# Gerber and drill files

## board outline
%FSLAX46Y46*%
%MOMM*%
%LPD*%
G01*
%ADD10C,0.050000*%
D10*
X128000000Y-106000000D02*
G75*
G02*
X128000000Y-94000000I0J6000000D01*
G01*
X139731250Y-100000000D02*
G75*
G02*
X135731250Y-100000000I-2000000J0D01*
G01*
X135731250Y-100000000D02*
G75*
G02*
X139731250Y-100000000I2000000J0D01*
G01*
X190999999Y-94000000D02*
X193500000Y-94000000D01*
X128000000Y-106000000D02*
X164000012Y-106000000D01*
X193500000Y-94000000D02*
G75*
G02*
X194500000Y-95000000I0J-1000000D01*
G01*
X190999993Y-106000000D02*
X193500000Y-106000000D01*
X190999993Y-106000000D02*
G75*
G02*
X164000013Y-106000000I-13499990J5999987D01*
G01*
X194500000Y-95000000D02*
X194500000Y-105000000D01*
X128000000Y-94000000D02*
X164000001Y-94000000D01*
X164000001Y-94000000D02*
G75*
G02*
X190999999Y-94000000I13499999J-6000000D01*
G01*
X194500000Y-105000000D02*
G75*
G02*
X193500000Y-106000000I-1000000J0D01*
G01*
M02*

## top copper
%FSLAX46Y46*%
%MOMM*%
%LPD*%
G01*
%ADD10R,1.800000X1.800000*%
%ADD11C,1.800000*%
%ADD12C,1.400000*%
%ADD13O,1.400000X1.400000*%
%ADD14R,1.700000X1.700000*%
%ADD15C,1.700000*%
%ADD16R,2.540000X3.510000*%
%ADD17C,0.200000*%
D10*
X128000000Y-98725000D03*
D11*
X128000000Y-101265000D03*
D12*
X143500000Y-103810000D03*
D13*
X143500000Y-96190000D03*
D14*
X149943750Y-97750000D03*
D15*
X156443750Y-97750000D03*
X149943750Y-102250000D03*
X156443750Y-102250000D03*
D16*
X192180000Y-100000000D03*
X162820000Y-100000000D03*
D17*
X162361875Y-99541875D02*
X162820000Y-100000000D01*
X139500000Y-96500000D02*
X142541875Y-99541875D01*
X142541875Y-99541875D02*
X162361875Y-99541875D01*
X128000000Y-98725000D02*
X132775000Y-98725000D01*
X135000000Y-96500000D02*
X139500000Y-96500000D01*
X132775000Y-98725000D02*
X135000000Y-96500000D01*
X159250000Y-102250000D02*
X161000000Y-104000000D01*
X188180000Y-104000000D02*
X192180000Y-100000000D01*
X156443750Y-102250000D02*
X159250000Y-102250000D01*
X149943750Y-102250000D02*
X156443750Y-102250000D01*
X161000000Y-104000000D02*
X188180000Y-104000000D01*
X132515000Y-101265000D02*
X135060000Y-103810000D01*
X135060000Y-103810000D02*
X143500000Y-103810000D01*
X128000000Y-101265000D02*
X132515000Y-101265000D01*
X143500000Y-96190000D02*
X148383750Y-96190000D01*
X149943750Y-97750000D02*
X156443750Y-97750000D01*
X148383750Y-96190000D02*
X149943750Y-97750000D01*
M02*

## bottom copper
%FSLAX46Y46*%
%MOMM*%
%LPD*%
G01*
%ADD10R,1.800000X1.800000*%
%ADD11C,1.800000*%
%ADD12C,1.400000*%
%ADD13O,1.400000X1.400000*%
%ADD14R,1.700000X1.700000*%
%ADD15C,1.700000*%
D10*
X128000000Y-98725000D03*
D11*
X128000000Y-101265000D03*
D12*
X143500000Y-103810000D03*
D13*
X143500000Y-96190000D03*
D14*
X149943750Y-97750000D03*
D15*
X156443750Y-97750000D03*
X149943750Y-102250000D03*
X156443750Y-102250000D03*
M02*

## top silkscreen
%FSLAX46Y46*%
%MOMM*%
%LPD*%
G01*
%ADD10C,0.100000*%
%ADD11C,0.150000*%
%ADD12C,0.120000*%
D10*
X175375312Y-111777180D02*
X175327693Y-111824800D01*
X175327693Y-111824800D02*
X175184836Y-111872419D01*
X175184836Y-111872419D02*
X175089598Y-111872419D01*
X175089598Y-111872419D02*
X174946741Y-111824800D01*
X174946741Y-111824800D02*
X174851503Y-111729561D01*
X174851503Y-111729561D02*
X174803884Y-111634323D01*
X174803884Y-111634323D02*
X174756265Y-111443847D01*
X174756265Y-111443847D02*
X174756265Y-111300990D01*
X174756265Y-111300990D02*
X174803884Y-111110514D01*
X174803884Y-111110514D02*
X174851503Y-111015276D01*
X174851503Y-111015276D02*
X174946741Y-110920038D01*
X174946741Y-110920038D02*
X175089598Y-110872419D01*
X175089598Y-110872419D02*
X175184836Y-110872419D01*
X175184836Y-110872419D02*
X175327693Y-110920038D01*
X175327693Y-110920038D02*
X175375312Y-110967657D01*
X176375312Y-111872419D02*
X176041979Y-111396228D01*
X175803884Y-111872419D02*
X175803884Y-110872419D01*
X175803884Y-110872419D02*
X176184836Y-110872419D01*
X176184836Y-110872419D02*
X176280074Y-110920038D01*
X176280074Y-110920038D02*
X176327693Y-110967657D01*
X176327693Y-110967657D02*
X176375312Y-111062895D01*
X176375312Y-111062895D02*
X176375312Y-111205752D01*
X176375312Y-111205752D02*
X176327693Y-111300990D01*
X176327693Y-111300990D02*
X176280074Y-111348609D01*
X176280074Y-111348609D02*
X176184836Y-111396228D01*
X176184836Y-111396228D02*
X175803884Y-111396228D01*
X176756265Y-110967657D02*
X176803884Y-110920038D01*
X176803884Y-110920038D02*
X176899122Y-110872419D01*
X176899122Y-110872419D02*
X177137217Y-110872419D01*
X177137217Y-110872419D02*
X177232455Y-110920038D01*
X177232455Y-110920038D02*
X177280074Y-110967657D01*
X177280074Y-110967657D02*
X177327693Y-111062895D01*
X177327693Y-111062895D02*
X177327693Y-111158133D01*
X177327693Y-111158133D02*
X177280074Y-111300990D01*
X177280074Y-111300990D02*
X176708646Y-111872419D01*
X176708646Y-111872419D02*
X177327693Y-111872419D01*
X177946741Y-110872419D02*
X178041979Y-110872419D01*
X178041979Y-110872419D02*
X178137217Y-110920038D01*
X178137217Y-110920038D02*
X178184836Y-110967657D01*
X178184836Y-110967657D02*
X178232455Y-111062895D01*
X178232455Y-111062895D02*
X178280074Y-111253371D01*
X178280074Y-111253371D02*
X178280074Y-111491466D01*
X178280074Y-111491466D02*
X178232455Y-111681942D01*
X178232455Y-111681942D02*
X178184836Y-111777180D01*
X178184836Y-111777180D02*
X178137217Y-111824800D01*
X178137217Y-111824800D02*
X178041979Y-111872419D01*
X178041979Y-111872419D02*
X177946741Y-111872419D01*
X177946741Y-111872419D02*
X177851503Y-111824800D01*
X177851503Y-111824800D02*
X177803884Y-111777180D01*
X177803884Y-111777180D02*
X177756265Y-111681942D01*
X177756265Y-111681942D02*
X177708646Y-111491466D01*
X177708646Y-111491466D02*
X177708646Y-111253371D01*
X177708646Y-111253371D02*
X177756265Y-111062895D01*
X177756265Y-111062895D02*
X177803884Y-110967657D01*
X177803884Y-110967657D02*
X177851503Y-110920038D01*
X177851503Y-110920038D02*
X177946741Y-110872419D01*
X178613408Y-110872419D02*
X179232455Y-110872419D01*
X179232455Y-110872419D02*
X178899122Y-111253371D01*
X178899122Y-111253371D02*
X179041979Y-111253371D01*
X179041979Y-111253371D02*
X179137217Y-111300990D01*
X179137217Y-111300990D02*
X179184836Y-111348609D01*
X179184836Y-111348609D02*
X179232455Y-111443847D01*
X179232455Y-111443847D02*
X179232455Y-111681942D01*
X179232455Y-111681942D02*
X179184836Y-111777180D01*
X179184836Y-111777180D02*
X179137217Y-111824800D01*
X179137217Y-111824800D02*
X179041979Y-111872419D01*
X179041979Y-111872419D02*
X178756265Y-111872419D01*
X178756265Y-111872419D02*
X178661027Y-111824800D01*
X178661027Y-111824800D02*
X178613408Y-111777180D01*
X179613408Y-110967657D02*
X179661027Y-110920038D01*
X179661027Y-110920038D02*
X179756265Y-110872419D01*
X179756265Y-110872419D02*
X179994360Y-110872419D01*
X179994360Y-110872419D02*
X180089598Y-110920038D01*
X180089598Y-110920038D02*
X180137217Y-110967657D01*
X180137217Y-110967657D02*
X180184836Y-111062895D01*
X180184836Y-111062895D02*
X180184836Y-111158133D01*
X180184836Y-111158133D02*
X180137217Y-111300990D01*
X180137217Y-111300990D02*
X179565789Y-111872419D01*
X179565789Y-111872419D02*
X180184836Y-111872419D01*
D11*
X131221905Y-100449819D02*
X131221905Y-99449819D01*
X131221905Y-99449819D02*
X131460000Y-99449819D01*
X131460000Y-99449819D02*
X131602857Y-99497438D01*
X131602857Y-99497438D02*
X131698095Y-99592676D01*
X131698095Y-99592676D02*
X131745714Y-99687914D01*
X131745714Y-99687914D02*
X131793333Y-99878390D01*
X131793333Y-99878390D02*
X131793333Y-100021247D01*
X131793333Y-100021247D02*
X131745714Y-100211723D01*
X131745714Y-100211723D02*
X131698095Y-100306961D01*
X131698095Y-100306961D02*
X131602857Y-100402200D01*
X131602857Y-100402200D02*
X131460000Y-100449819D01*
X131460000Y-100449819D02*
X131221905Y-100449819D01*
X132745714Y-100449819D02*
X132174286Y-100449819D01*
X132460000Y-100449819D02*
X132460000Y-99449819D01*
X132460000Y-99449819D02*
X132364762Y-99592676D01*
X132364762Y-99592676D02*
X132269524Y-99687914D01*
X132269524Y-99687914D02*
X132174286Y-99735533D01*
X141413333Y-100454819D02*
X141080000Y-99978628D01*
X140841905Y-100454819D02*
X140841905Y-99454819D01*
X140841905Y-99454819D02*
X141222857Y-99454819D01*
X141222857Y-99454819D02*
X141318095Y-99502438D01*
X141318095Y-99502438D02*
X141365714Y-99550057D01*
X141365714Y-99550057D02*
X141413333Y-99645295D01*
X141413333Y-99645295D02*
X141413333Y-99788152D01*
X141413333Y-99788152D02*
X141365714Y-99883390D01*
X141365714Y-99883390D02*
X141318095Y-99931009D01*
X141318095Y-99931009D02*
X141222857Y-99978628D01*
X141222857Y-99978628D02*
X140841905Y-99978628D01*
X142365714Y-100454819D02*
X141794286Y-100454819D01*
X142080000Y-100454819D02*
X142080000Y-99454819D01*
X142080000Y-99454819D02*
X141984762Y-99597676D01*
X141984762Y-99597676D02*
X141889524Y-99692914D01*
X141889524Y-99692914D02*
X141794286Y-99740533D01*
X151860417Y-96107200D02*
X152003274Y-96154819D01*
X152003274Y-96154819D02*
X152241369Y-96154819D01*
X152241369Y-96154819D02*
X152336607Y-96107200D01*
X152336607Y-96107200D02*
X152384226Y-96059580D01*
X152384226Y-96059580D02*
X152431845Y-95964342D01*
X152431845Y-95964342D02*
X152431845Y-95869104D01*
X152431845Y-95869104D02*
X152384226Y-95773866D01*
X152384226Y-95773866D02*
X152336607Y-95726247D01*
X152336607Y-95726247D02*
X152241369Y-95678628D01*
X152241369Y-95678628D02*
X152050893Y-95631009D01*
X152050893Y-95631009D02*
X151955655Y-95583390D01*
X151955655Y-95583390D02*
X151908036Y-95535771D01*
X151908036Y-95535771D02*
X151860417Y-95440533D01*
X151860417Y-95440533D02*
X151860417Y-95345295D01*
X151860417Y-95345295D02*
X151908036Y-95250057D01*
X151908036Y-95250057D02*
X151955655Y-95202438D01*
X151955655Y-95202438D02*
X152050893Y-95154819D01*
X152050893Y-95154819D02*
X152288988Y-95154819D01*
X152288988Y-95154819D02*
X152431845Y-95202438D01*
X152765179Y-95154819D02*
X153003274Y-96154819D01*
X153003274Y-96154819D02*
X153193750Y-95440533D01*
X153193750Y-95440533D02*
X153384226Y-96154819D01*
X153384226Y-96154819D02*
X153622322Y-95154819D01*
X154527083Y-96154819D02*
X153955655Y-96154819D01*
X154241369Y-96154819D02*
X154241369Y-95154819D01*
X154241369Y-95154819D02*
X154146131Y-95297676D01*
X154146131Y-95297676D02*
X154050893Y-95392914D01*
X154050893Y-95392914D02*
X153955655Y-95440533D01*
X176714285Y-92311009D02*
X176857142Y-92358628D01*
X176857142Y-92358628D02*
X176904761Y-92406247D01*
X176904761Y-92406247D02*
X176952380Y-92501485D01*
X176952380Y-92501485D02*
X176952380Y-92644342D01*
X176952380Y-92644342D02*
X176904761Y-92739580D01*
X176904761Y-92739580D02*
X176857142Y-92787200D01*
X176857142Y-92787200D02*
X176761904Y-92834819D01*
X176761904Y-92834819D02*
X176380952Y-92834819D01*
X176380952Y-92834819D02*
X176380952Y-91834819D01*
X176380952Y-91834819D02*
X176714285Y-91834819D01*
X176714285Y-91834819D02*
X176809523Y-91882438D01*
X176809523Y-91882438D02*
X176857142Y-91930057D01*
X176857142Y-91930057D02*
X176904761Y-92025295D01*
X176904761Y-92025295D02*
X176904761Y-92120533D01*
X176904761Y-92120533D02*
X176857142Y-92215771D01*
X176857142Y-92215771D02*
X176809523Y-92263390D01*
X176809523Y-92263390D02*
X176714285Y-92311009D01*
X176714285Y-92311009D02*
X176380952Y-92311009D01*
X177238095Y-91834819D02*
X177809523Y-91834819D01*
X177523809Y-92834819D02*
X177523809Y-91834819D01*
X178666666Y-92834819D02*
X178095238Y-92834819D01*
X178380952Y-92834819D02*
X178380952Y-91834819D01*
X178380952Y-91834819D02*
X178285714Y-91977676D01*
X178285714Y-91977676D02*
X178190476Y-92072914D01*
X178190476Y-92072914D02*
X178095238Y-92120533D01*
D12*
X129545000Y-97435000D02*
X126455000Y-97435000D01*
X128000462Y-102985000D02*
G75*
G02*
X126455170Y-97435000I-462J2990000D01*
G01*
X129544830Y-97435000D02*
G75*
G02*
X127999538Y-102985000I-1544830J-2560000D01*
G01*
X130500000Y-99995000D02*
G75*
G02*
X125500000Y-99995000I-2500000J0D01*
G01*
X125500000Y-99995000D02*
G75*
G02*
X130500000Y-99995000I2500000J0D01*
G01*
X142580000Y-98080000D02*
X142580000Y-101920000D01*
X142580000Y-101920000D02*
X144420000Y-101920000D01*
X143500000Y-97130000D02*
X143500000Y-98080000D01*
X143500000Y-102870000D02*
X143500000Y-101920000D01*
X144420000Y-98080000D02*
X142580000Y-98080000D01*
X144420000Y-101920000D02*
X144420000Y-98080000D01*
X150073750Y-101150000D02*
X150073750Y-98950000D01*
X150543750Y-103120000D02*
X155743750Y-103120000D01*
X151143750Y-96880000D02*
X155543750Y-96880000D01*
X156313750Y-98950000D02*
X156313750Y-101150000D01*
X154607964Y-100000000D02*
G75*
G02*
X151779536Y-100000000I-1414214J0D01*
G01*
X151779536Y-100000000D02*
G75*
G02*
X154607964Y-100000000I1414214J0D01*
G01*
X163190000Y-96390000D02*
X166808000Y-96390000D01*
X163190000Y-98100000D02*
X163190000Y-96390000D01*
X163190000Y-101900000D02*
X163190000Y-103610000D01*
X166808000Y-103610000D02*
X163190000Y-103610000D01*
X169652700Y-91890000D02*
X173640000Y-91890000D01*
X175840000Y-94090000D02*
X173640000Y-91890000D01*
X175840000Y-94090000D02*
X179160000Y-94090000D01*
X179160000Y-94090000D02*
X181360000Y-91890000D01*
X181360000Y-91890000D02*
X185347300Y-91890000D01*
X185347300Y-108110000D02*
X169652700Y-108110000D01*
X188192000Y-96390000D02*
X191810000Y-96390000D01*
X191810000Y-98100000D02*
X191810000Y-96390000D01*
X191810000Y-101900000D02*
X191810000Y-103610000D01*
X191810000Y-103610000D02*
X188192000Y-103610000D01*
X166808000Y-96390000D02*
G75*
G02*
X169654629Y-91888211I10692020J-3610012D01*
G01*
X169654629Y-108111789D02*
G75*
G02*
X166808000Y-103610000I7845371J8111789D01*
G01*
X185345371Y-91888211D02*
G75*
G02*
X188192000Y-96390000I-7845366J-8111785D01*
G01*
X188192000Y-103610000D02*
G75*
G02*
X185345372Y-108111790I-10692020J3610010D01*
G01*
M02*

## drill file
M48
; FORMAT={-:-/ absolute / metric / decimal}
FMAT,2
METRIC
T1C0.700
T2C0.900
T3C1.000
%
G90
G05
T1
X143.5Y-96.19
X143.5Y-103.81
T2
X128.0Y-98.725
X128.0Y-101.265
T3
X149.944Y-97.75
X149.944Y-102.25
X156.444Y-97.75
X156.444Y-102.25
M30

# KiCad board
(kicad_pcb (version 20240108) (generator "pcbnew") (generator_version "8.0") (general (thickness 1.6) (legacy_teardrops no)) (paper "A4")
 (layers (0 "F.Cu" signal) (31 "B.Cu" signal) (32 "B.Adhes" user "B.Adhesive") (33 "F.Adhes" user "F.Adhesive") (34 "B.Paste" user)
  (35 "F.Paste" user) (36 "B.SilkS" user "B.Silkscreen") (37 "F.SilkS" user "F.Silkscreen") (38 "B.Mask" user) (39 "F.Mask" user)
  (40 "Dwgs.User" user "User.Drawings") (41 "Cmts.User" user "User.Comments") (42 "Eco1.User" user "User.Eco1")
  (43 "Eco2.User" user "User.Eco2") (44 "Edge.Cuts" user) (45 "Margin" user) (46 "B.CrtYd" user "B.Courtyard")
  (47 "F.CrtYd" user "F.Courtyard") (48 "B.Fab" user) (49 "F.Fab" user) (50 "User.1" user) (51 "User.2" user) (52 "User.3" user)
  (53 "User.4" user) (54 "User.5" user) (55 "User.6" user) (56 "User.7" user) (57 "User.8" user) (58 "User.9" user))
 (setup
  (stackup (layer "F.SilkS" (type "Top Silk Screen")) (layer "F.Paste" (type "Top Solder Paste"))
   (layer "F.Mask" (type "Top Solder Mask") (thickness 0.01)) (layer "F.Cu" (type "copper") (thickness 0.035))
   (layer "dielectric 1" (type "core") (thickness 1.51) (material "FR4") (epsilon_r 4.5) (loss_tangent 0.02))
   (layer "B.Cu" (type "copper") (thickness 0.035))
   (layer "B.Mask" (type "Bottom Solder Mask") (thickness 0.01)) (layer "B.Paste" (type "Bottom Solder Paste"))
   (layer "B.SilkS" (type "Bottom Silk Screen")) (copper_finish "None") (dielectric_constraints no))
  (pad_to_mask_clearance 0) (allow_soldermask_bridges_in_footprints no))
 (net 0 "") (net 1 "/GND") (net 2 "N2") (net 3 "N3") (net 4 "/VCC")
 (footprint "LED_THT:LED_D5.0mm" (layer "F.Cu") (at 128 98.725 -90)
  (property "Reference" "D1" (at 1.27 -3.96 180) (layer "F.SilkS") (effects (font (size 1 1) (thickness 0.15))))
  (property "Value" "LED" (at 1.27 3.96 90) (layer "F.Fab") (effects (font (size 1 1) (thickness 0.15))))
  (fp_line (start -1.29 -1.545) (end -1.29 1.545) (stroke (width 0.12) (type solid)) (layer "F.SilkS"))
  (fp_arc (start 4.26 -0.000462) (mid 2.072002 2.880433) (end -1.29 1.54483) (stroke (width 0.12) (type solid)) (layer "F.SilkS"))
  (fp_arc (start -1.29 -1.54483) (mid 2.072002 -2.880433) (end 4.26 0.000462) (stroke (width 0.12) (type solid)) (layer "F.SilkS"))
  (fp_circle (center 1.27 0) (end 3.77 0) (stroke (width 0.12) (type solid)) (fill none) (layer "F.SilkS"))
  (pad "1" thru_hole rect (at 0 0 270) (size 1.8 1.8) (drill 0.9) (layers "*.Cu" "*.Mask") (remove_unused_layers no) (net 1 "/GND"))
  (pad "2" thru_hole circle (at 2.54 0 270) (size 1.8 1.8) (drill 0.9) (layers "*.Cu" "*.Mask") (remove_unused_layers no) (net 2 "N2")))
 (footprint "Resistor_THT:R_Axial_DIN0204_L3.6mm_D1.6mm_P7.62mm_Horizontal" (layer "F.Cu") (at 143.5 103.81 90)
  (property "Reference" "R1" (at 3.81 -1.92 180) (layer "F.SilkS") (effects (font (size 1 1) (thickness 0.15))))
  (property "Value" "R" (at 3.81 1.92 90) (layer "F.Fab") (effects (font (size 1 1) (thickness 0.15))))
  (fp_line (start 5.73 -0.92) (end 1.89 -0.92) (stroke (width 0.12) (type solid)) (layer "F.SilkS"))
  (fp_line (start 1.89 -0.92) (end 1.89 0.92) (stroke (width 0.12) (type solid)) (layer "F.SilkS"))
  (fp_line (start 6.68 0) (end 5.73 0) (stroke (width 0.12) (type solid)) (layer "F.SilkS"))
  (fp_line (start 0.94 0) (end 1.89 0) (stroke (width 0.12) (type solid)) (layer "F.SilkS"))
  (fp_line (start 5.73 0.92) (end 5.73 -0.92) (stroke (width 0.12) (type solid)) (layer "F.SilkS"))
  (fp_line (start 1.89 0.92) (end 5.73 0.92) (stroke (width 0.12) (type solid)) (layer "F.SilkS"))
  (pad "1" thru_hole circle (at 0 0 90) (size 1.4 1.4) (drill 0.7) (layers "*.Cu" "*.Mask") (remove_unused_layers no) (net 2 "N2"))
  (pad "2" thru_hole oval (at 7.62 0 90) (size 1.4 1.4) (drill 0.7) (layers "*.Cu" "*.Mask") (remove_unused_layers no) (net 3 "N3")))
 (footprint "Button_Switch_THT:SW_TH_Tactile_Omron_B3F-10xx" (layer "F.Cu") (at 149.94375 97.75)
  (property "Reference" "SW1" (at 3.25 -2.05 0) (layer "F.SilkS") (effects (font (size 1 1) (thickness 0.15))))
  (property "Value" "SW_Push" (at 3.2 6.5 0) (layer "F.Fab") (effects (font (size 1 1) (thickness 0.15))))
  (fp_line (start 0.13 3.4) (end 0.13 1.2) (stroke (width 0.12) (type solid)) (layer "F.SilkS"))
  (fp_line (start 0.6 5.37) (end 5.8 5.37) (stroke (width 0.12) (type solid)) (layer "F.SilkS"))
  (fp_line (start 1.2 -0.87) (end 5.6 -0.87) (stroke (width 0.12) (type solid)) (layer "F.SilkS"))
  (fp_line (start 6.37 1.2) (end 6.37 3.4) (stroke (width 0.12) (type solid)) (layer "F.SilkS"))
  (fp_circle (center 3.25 2.25) (end 4.25 3.25) (stroke (width 0.12) (type solid)) (fill none) (layer "F.SilkS"))
  (pad "1" thru_hole rect (at 0 0) (size 1.7 1.7) (drill 1) (layers "*.Cu" "*.Mask") (remove_unused_layers no) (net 3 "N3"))
  (pad "1" thru_hole circle (at 6.5 0) (size 1.7 1.7) (drill 1) (layers "*.Cu" "*.Mask") (remove_unused_layers no) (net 3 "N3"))
  (pad "2" thru_hole circle (at 0 4.5) (size 1.7 1.7) (drill 1) (layers "*.Cu" "*.Mask") (remove_unused_layers no) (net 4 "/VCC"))
  (pad "2" thru_hole circle (at 6.5 4.5) (size 1.7 1.7) (drill 1) (layers "*.Cu" "*.Mask") (remove_unused_layers no) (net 4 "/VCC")))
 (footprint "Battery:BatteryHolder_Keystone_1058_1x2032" (layer "F.Cu") (at 177.5 100 180)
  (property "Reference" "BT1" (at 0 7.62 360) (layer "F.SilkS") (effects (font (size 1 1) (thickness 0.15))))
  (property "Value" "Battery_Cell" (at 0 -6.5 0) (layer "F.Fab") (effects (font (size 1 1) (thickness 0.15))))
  (fp_line (start 14.31 3.61) (end 10.692 3.61) (stroke (width 0.12) (type solid)) (layer "F.SilkS"))
  (fp_line (start 14.31 1.9) (end 14.31 3.61) (stroke (width 0.12) (type solid)) (layer "F.SilkS"))
  (fp_line (start 14.31 -1.9) (end 14.31 -3.61) (stroke (width 0.12) (type solid)) (layer "F.SilkS"))
  (fp_line (start 10.692 -3.61) (end 14.31 -3.61) (stroke (width 0.12) (type solid)) (layer "F.SilkS"))
  (fp_line (start 7.8473 8.11) (end 3.86 8.11) (stroke (width 0.12) (type solid)) (layer "F.SilkS"))
  (fp_line (start 1.66 5.91) (end 3.86 8.11) (stroke (width 0.12) (type solid)) (layer "F.SilkS"))
  (fp_line (start 1.66 5.91) (end -1.66 5.91) (stroke (width 0.12) (type solid)) (layer "F.SilkS"))
  (fp_line (start -1.66 5.91) (end -3.86 8.11) (stroke (width 0.12) (type solid)) (layer "F.SilkS"))
  (fp_line (start -3.86 8.11) (end -7.8473 8.11) (stroke (width 0.12) (type solid)) (layer "F.SilkS"))
  (fp_line (start -7.8473 -8.11) (end 7.8473 -8.11) (stroke (width 0.12) (type solid)) (layer "F.SilkS"))
  (fp_line (start -10.692 3.61) (end -14.31 3.61) (stroke (width 0.12) (type solid)) (layer "F.SilkS"))
  (fp_line (start -14.31 1.9) (end -14.31 3.61) (stroke (width 0.12) (type solid)) (layer "F.SilkS"))
  (fp_line (start -14.31 -1.9) (end -14.31 -3.61) (stroke (width 0.12) (type solid)) (layer "F.SilkS"))
  (fp_line (start -14.31 -3.61) (end -10.692 -3.61) (stroke (width 0.12) (type solid)) (layer "F.SilkS"))
  (fp_arc (start 10.692 3.61) (mid 9.538084 6.031244) (end 7.845371 8.111789) (stroke (width 0.12) (type solid)) (layer "F.SilkS"))
  (fp_arc (start 7.845371 -8.111789) (mid 9.538085 -6.031244) (end 10.692 -3.61) (stroke (width 0.12) (type solid)) (layer "F.SilkS"))
  (fp_arc (start -7.845371 8.111789) (mid -9.538085 6.031244) (end -10.692 3.61) (stroke (width 0.12) (type solid)) (layer "F.SilkS"))
  (fp_arc (start -10.692 -3.61) (mid -9.538084 -6.031244) (end -7.845371 -8.111789) (stroke (width 0.12) (type solid)) (layer "F.SilkS"))
  (pad "1" smd rect (at -14.68 0 180) (size 2.54 3.51) (layers "F.Cu" "F.Paste" "F.Mask") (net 4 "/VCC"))
  (pad "2" smd rect (at 14.68 0 180) (size 2.54 3.51) (layers "F.Cu" "F.Paste" "F.Mask") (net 1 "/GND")))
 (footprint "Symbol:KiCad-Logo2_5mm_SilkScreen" (layer "B.Cu") (at 177.5 100 180)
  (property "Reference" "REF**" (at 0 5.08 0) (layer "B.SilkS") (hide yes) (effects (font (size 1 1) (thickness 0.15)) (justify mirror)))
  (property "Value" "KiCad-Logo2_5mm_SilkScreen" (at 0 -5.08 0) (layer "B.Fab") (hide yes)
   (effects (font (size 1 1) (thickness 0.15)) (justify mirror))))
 (gr_arc (start 128 106) (mid 122 100) (end 128 94) (locked yes) (stroke (width 0.05) (type default)) (layer "Edge.Cuts"))
 (gr_circle (center 137.73125 100) (end 137.73125 102) (stroke (width 0.05) (type default)) (fill none) (layer "Edge.Cuts"))
 (gr_line (start 190.999999 94) (end 193.5 94) (locked yes) (stroke (width 0.05) (type default)) (layer "Edge.Cuts"))
 (gr_line (start 128 106) (end 164.000012 106) (locked yes) (stroke (width 0.05) (type default)) (layer "Edge.Cuts"))
 (gr_arc (start 193.5 94) (mid 194.207107 94.292893) (end 194.5 95) (locked yes) (stroke (width 0.05) (type default)) (layer "Edge.Cuts"))
 (gr_line (start 190.999993 106) (end 193.5 106) (locked yes) (stroke (width 0.05) (type default)) (layer "Edge.Cuts"))
 (gr_arc (start 190.999993 106) (mid 177.500001 114.773286) (end 164.000012 106) (locked yes) (stroke (width 0.05) (type default))
  (layer "Edge.Cuts"))
 (gr_line (start 194.5 95) (end 194.5 105) (locked yes) (stroke (width 0.05) (type default)) (layer "Edge.Cuts"))
 (gr_line (start 128 94) (end 164.000001 94) (locked yes) (stroke (width 0.05) (type default)) (layer "Edge.Cuts"))
 (gr_arc (start 164.000001 94) (mid 177.5 85.226714) (end 190.999999 94) (locked yes) (stroke (width 0.05) (type default))
  (layer "Edge.Cuts"))
 (gr_arc (start 194.5 105) (mid 194.207107 105.707107) (end 193.5 106) (locked yes) (stroke (width 0.05) (type default)) (layer "Edge.Cuts"))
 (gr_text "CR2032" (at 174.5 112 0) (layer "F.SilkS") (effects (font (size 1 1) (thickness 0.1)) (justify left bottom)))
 (segment (start 162.361875 99.541875) (end 162.82 100) (width 0.2) (layer "F.Cu") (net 1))
 (segment (start 139.5 96.5) (end 142.541875 99.541875) (width 0.2) (layer "F.Cu") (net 1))
 (segment (start 142.541875 99.541875) (end 162.361875 99.541875) (width 0.2) (layer "F.Cu") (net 1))
 (segment (start 128 98.725) (end 132.775 98.725) (width 0.2) (layer "F.Cu") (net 1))
 (segment (start 135 96.5) (end 139.5 96.5) (width 0.2) (layer "F.Cu") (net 1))
 (segment (start 132.775 98.725) (end 135 96.5) (width 0.2) (layer "F.Cu") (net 1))
 (segment (start 159.25 102.25) (end 161 104) (width 0.2) (layer "F.Cu") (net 4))
 (segment (start 188.18 104) (end 192.18 100) (width 0.2) (layer "F.Cu") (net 4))
 (segment (start 156.44375 102.25) (end 159.25 102.25) (width 0.2) (layer "F.Cu") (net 4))
 (segment (start 149.94375 102.25) (end 156.44375 102.25) (width 0.2) (layer "F.Cu") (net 4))
 (segment (start 161 104) (end 188.18 104) (width 0.2) (layer "F.Cu") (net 4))
 (segment (start 132.515 101.265) (end 135.06 103.81) (width 0.2) (layer "F.Cu") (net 2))
 (segment (start 135.06 103.81) (end 143.5 103.81) (width 0.2) (layer "F.Cu") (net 2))
 (segment (start 128 101.265) (end 132.515 101.265) (width 0.2) (layer "F.Cu") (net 2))
 (segment (start 143.5 96.19) (end 148.38375 96.19) (width 0.2) (layer "F.Cu") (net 3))
 (segment (start 149.94375 97.75) (end 156.44375 97.75) (width 0.2) (layer "F.Cu") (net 3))
 (segment (start 148.38375 96.19) (end 149.94375 97.75) (width 0.2) (layer "F.Cu") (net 3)))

